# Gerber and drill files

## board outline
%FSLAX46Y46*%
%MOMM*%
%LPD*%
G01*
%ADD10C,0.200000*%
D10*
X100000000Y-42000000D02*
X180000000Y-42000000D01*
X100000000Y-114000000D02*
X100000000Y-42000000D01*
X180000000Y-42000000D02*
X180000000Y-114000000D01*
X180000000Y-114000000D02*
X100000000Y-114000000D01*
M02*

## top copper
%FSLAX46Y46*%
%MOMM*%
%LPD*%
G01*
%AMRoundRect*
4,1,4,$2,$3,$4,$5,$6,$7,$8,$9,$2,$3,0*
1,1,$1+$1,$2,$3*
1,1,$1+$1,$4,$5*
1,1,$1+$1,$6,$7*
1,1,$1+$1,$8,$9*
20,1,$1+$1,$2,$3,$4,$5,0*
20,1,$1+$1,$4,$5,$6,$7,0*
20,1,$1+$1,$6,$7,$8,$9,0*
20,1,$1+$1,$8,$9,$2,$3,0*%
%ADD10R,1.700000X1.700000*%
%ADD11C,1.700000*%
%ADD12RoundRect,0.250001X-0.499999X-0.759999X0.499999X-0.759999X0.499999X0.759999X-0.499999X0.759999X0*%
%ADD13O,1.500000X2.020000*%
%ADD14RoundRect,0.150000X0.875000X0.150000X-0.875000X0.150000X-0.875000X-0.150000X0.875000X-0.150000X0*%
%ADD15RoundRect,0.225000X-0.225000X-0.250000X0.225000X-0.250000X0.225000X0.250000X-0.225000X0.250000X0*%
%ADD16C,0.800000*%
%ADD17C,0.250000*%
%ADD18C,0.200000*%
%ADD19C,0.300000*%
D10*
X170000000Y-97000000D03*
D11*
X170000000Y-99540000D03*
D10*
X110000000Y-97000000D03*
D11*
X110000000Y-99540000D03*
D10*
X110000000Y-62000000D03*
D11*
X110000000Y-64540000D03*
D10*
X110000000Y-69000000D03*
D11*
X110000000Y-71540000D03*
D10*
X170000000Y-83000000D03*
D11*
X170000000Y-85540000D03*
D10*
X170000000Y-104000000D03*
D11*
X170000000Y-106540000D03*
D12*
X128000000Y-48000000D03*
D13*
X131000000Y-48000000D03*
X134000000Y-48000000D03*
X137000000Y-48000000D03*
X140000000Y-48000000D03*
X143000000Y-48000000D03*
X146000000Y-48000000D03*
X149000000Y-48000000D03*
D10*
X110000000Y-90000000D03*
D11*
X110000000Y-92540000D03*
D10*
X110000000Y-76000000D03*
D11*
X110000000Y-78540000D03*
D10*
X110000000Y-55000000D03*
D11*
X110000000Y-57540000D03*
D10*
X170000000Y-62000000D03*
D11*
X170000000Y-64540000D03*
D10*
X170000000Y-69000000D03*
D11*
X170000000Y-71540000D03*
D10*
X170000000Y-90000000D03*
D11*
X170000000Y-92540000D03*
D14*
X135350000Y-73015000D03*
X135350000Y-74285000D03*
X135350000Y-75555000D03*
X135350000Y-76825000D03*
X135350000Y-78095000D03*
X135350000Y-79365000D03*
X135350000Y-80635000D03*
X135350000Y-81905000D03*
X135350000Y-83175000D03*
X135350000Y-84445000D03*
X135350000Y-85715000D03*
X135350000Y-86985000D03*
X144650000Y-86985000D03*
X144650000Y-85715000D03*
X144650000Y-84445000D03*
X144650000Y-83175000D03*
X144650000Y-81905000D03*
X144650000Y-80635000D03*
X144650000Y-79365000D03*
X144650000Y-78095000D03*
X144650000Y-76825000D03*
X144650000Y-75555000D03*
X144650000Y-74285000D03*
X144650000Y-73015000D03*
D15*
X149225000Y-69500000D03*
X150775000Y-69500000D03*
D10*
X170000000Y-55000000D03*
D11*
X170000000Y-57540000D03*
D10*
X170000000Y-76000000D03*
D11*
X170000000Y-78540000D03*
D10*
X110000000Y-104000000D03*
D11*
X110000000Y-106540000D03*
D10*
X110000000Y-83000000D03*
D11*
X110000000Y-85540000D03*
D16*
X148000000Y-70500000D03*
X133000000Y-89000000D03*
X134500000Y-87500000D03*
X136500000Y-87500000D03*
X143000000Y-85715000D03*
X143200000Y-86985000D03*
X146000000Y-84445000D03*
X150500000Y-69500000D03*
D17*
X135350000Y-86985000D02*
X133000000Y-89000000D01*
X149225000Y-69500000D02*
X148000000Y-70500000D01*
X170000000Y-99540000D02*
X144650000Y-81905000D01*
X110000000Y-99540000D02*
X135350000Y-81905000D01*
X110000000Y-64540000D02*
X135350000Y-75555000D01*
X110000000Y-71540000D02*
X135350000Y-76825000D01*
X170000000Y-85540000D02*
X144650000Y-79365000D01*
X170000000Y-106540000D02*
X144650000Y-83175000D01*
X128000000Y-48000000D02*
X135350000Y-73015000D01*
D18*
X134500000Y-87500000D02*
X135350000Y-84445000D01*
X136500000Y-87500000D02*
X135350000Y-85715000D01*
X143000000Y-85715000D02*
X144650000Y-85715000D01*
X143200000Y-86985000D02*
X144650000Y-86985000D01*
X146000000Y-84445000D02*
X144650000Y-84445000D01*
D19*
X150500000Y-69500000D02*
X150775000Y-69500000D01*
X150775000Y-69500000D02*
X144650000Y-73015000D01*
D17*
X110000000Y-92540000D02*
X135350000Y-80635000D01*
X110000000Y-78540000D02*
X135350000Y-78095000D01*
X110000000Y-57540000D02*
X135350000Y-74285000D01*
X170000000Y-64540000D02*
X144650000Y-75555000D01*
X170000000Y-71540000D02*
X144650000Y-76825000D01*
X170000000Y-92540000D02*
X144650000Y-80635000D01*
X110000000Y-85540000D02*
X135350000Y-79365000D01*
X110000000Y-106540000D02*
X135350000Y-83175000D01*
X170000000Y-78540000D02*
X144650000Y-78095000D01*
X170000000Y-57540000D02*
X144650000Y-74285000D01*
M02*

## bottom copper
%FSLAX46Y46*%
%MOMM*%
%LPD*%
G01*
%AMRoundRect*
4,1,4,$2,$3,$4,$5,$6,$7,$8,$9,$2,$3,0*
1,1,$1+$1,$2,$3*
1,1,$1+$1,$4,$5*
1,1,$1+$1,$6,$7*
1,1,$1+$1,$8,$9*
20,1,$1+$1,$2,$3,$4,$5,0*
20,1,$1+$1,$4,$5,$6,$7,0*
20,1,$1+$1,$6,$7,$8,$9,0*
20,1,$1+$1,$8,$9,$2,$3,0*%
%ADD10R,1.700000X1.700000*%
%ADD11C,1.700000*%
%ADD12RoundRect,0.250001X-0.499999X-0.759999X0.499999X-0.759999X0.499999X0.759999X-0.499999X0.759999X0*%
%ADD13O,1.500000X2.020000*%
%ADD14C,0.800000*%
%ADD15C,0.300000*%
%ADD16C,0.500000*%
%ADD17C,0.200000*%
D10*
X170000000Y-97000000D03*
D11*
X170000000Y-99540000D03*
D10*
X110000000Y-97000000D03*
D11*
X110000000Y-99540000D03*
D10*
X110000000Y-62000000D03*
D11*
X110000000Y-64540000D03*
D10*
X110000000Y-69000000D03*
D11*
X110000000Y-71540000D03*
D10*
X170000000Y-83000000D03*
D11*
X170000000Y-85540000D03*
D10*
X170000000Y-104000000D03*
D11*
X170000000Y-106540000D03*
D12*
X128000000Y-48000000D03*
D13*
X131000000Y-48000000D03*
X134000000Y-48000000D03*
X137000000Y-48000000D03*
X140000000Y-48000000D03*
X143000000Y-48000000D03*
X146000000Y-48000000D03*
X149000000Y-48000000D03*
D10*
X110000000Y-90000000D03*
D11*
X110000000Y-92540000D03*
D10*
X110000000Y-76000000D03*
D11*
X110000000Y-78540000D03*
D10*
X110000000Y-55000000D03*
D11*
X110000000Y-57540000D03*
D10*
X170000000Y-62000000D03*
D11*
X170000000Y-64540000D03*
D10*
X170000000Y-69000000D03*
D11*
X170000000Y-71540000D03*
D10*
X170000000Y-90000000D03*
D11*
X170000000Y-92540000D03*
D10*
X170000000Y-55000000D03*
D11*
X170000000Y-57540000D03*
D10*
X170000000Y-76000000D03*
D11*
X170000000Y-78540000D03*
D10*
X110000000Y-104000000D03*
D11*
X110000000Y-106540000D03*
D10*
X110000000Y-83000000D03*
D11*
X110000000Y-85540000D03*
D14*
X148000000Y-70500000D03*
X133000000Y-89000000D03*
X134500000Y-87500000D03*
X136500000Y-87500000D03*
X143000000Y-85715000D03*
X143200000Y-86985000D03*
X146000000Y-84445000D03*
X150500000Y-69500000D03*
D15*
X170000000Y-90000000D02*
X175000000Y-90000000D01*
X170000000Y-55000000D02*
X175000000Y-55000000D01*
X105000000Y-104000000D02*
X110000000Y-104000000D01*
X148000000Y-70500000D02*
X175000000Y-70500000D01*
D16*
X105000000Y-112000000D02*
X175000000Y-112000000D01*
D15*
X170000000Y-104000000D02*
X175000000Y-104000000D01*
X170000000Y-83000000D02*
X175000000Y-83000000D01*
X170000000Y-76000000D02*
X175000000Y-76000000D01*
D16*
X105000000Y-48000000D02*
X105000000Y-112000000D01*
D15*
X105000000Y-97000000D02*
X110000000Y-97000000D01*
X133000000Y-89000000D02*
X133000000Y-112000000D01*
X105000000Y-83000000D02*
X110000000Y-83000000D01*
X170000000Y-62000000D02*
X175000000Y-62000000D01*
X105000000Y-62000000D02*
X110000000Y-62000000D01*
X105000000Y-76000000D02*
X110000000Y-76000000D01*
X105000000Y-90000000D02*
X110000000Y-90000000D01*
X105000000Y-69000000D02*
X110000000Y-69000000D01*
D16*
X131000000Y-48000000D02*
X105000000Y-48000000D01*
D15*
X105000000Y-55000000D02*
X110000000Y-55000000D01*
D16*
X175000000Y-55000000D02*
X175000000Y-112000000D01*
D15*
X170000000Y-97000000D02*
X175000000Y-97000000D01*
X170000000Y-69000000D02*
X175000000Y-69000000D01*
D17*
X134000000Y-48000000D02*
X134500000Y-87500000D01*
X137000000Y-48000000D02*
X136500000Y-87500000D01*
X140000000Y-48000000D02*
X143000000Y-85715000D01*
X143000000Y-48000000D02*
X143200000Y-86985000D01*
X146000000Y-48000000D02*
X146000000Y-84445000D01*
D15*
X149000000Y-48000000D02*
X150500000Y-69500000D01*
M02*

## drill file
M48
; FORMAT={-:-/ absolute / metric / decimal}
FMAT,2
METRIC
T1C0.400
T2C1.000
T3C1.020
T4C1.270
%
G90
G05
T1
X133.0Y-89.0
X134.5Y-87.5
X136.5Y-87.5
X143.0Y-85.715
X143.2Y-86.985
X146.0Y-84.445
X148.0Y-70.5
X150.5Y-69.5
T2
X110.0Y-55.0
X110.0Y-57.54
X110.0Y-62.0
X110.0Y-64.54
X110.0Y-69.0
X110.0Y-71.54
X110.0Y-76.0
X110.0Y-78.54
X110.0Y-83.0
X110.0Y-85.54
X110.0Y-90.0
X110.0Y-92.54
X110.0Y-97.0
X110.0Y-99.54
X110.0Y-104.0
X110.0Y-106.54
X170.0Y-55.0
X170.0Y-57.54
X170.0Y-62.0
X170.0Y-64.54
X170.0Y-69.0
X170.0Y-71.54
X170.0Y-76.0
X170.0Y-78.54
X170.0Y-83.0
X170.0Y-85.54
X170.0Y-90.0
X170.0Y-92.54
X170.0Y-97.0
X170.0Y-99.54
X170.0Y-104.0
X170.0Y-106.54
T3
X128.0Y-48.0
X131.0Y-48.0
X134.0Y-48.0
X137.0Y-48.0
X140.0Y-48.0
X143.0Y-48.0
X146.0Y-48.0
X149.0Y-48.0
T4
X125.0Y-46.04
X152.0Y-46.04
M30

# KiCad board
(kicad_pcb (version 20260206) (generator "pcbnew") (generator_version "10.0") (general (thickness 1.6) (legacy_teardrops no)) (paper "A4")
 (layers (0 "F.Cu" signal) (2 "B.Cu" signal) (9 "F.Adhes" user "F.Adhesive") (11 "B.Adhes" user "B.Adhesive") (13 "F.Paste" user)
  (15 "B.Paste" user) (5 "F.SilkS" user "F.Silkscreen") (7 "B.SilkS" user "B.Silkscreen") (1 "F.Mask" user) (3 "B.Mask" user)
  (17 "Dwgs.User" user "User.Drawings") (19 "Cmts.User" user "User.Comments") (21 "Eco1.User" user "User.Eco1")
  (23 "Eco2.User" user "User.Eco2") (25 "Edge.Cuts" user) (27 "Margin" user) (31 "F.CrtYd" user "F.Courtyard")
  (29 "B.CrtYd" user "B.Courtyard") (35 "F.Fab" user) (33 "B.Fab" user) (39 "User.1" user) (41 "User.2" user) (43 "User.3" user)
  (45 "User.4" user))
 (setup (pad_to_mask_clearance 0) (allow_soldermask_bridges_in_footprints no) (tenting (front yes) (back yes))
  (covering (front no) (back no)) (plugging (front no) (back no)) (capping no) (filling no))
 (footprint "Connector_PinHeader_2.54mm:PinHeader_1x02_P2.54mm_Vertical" (layer "F.Cu") (at 170 97)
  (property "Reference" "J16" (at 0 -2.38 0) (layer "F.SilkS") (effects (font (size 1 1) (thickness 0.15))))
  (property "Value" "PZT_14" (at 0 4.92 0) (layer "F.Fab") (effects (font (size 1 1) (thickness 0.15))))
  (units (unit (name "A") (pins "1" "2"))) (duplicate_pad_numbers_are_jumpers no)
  (pad "1" thru_hole rect (at 0 0) (size 1.7 1.7) (drill 1) (layers "*.Cu" "*.Mask") (remove_unused_layers no) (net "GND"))
  (pad "2" thru_hole circle (at 0 2.54) (size 1.7 1.7) (drill 1) (layers "*.Cu" "*.Mask") (remove_unused_layers no) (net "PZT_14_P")))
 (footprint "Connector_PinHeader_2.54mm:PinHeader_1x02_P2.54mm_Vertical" (layer "F.Cu") (at 110 97)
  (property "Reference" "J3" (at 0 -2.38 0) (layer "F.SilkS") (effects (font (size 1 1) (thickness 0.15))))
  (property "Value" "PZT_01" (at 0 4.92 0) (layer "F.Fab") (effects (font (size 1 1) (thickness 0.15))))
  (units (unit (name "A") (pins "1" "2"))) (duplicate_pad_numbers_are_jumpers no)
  (pad "1" thru_hole rect (at 0 0) (size 1.7 1.7) (drill 1) (layers "*.Cu" "*.Mask") (remove_unused_layers no) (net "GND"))
  (pad "2" thru_hole circle (at 0 2.54) (size 1.7 1.7) (drill 1) (layers "*.Cu" "*.Mask") (remove_unused_layers no) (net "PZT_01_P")))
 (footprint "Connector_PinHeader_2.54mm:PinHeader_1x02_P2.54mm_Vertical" (layer "F.Cu") (at 110 62)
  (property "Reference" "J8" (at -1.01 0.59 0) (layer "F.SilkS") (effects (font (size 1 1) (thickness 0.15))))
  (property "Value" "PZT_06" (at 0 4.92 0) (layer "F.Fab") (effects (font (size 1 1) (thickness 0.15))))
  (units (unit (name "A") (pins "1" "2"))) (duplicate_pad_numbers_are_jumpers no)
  (pad "1" thru_hole rect (at 0 0) (size 1.7 1.7) (drill 1) (layers "*.Cu" "*.Mask") (remove_unused_layers no) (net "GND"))
  (pad "2" thru_hole circle (at 0 2.54) (size 1.7 1.7) (drill 1) (layers "*.Cu" "*.Mask") (remove_unused_layers no) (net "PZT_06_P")))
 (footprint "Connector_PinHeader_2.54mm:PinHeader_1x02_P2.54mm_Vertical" (layer "F.Cu") (at 110 69)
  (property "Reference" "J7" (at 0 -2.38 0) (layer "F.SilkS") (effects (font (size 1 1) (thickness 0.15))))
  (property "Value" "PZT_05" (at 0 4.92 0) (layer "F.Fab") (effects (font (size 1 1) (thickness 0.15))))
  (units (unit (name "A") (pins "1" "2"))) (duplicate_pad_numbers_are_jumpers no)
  (pad "1" thru_hole rect (at 0 0) (size 1.7 1.7) (drill 1) (layers "*.Cu" "*.Mask") (remove_unused_layers no) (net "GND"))
  (pad "2" thru_hole circle (at 0 2.54) (size 1.7 1.7) (drill 1) (layers "*.Cu" "*.Mask") (remove_unused_layers no) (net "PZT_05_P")))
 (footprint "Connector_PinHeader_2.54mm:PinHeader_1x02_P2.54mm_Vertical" (layer "F.Cu") (at 170 83)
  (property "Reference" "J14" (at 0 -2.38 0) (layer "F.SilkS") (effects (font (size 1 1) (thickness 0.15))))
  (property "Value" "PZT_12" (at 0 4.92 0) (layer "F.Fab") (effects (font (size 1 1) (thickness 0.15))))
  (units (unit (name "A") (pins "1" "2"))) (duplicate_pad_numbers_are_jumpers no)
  (pad "1" thru_hole rect (at 0 0) (size 1.7 1.7) (drill 1) (layers "*.Cu" "*.Mask") (remove_unused_layers no) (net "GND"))
  (pad "2" thru_hole circle (at 0 2.54) (size 1.7 1.7) (drill 1) (layers "*.Cu" "*.Mask") (remove_unused_layers no) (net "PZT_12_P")))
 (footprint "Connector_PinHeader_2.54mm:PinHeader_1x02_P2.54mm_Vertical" (layer "F.Cu") (at 170 104)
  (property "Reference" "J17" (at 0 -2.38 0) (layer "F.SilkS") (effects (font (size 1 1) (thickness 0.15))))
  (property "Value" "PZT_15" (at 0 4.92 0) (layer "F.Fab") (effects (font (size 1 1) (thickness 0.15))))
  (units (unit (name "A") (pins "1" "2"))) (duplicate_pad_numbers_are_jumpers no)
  (pad "1" thru_hole rect (at 0 0) (size 1.7 1.7) (drill 1) (layers "*.Cu" "*.Mask") (remove_unused_layers no) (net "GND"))
  (pad "2" thru_hole circle (at 0 2.54) (size 1.7 1.7) (drill 1) (layers "*.Cu" "*.Mask") (remove_unused_layers no) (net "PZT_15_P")))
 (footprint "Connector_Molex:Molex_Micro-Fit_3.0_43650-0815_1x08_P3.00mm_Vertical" (layer "F.Cu") (at 128 48)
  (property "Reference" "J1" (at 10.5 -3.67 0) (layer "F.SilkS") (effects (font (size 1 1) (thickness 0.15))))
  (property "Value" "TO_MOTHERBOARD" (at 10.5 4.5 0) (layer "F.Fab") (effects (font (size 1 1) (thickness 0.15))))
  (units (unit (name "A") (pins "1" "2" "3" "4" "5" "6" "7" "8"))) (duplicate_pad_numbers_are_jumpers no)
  (pad "" np_thru_hole circle (at -3 -1.96) (size 1.27 1.27) (drill 1.27) (layers "*.Cu" "*.Mask"))
  (pad "" np_thru_hole circle (at 24 -1.96) (size 1.27 1.27) (drill 1.27) (layers "*.Cu" "*.Mask"))
  (pad "1" thru_hole roundrect (at 0 0) (size 1.5 2.02) (drill 1.02) (layers "*.Cu" "*.Mask") (remove_unused_layers no)
   (roundrect_rratio 0.166667) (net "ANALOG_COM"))
  (pad "2" thru_hole oval (at 3 0) (size 1.5 2.02) (drill 1.02) (layers "*.Cu" "*.Mask") (remove_unused_layers no) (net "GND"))
  (pad "3" thru_hole oval (at 6 0) (size 1.5 2.02) (drill 1.02) (layers "*.Cu" "*.Mask") (remove_unused_layers no) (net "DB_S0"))
  (pad "4" thru_hole oval (at 9 0) (size 1.5 2.02) (drill 1.02) (layers "*.Cu" "*.Mask") (remove_unused_layers no) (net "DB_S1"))
  (pad "5" thru_hole oval (at 12 0) (size 1.5 2.02) (drill 1.02) (layers "*.Cu" "*.Mask") (remove_unused_layers no) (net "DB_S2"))
  (pad "6" thru_hole oval (at 15 0) (size 1.5 2.02) (drill 1.02) (layers "*.Cu" "*.Mask") (remove_unused_layers no) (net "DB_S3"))
  (pad "7" thru_hole oval (at 18 0) (size 1.5 2.02) (drill 1.02) (layers "*.Cu" "*.Mask") (remove_unused_layers no) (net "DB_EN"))
  (pad "8" thru_hole oval (at 21 0) (size 1.5 2.02) (drill 1.02) (layers "*.Cu" "*.Mask") (remove_unused_layers no) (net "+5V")))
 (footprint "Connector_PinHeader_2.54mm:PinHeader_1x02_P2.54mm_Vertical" (layer "F.Cu") (at 110 90)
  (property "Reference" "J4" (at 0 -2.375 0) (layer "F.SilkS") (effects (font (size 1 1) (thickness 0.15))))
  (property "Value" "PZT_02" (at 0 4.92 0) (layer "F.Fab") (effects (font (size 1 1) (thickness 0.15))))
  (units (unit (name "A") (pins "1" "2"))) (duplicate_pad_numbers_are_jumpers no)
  (pad "1" thru_hole rect (at 0 0) (size 1.7 1.7) (drill 1) (layers "*.Cu" "*.Mask") (remove_unused_layers no) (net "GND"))
  (pad "2" thru_hole circle (at 0 2.54) (size 1.7 1.7) (drill 1) (layers "*.Cu" "*.Mask") (remove_unused_layers no) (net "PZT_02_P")))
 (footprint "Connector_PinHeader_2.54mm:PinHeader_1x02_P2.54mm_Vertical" (layer "F.Cu") (at 110 76)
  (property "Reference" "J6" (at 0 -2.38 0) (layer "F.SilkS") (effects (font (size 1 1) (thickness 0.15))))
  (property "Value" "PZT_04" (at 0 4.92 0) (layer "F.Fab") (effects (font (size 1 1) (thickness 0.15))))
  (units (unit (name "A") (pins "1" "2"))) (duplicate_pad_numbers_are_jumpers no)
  (pad "1" thru_hole rect (at 0 0) (size 1.7 1.7) (drill 1) (layers "*.Cu" "*.Mask") (remove_unused_layers no) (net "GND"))
  (pad "2" thru_hole circle (at 0 2.54) (size 1.7 1.7) (drill 1) (layers "*.Cu" "*.Mask") (remove_unused_layers no) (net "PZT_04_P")))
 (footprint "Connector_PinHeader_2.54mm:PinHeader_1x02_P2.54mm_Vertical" (layer "F.Cu") (at 110 55)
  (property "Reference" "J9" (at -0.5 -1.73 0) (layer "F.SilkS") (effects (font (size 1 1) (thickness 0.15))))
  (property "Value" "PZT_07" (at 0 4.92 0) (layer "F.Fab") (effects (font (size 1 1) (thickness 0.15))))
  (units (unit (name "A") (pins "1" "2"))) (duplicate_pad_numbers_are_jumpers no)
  (pad "1" thru_hole rect (at 0 0) (size 1.7 1.7) (drill 1) (layers "*.Cu" "*.Mask") (remove_unused_layers no) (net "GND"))
  (pad "2" thru_hole circle (at 0 2.54) (size 1.7 1.7) (drill 1) (layers "*.Cu" "*.Mask") (remove_unused_layers no) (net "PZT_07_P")))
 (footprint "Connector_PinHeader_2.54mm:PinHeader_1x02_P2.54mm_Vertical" (layer "F.Cu") (at 170 62)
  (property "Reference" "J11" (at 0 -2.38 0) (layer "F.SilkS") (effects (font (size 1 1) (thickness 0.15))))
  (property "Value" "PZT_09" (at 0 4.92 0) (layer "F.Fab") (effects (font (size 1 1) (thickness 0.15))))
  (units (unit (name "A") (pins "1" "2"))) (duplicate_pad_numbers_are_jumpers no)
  (pad "1" thru_hole rect (at 0 0) (size 1.7 1.7) (drill 1) (layers "*.Cu" "*.Mask") (remove_unused_layers no) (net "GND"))
  (pad "2" thru_hole circle (at 0 2.54) (size 1.7 1.7) (drill 1) (layers "*.Cu" "*.Mask") (remove_unused_layers no) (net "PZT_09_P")))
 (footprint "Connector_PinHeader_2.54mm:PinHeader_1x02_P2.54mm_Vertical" (layer "F.Cu") (at 170 69)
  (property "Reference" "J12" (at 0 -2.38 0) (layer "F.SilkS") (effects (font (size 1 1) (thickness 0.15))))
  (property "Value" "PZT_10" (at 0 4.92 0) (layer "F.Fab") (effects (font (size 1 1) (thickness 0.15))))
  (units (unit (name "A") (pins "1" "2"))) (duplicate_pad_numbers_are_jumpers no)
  (pad "1" thru_hole rect (at 0 0) (size 1.7 1.7) (drill 1) (layers "*.Cu" "*.Mask") (remove_unused_layers no) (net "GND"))
  (pad "2" thru_hole circle (at 0 2.54) (size 1.7 1.7) (drill 1) (layers "*.Cu" "*.Mask") (remove_unused_layers no) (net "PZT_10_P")))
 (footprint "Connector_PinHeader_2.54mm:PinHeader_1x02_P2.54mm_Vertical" (layer "F.Cu") (at 170 90)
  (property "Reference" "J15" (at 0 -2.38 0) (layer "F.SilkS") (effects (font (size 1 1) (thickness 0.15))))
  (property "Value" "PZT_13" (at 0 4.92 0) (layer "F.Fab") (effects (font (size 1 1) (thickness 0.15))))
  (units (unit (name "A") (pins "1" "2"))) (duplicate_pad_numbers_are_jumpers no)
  (pad "1" thru_hole rect (at 0 0) (size 1.7 1.7) (drill 1) (layers "*.Cu" "*.Mask") (remove_unused_layers no) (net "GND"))
  (pad "2" thru_hole circle (at 0 2.54) (size 1.7 1.7) (drill 1) (layers "*.Cu" "*.Mask") (remove_unused_layers no) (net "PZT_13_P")))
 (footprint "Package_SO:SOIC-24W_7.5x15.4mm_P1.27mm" (layer "F.Cu") (at 140 80)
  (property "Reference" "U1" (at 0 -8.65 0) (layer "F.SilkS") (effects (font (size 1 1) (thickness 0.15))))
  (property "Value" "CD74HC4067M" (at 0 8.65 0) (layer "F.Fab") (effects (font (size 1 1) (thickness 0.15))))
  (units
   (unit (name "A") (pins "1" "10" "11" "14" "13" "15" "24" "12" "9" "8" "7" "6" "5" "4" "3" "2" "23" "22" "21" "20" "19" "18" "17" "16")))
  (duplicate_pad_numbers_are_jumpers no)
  (pad "1" smd roundrect (at -4.65 -6.985 180) (size 2.05 0.6) (layers "F.Cu" "F.Mask" "F.Paste") (roundrect_rratio 0.25) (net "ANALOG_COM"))
  (pad "2" smd roundrect (at -4.65 -5.715 180) (size 2.05 0.6) (layers "F.Cu" "F.Mask" "F.Paste") (roundrect_rratio 0.25) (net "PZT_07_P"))
  (pad "3" smd roundrect (at -4.65 -4.445 180) (size 2.05 0.6) (layers "F.Cu" "F.Mask" "F.Paste") (roundrect_rratio 0.25) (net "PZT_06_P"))
  (pad "4" smd roundrect (at -4.65 -3.175 180) (size 2.05 0.6) (layers "F.Cu" "F.Mask" "F.Paste") (roundrect_rratio 0.25) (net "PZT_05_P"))
  (pad "5" smd roundrect (at -4.65 -1.905 180) (size 2.05 0.6) (layers "F.Cu" "F.Mask" "F.Paste") (roundrect_rratio 0.25) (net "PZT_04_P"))
  (pad "6" smd roundrect (at -4.65 -0.635 180) (size 2.05 0.6) (layers "F.Cu" "F.Mask" "F.Paste") (roundrect_rratio 0.25) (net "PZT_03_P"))
  (pad "7" smd roundrect (at -4.65 0.635 180) (size 2.05 0.6) (layers "F.Cu" "F.Mask" "F.Paste") (roundrect_rratio 0.25) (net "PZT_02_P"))
  (pad "8" smd roundrect (at -4.65 1.905 180) (size 2.05 0.6) (layers "F.Cu" "F.Mask" "F.Paste") (roundrect_rratio 0.25) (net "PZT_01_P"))
  (pad "9" smd roundrect (at -4.65 3.175 180) (size 2.05 0.6) (layers "F.Cu" "F.Mask" "F.Paste") (roundrect_rratio 0.25) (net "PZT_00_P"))
  (pad "10" smd roundrect (at -4.65 4.445 180) (size 2.05 0.6) (layers "F.Cu" "F.Mask" "F.Paste") (roundrect_rratio 0.25) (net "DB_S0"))
  (pad "11" smd roundrect (at -4.65 5.715 180) (size 2.05 0.6) (layers "F.Cu" "F.Mask" "F.Paste") (roundrect_rratio 0.25) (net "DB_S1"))
  (pad "12" smd roundrect (at -4.65 6.985 180) (size 2.05 0.6) (layers "F.Cu" "F.Mask" "F.Paste") (roundrect_rratio 0.25) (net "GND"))
  (pad "13" smd roundrect (at 4.65 6.985 180) (size 2.05 0.6) (layers "F.Cu" "F.Mask" "F.Paste") (roundrect_rratio 0.25) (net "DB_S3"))
  (pad "14" smd roundrect (at 4.65 5.715 180) (size 2.05 0.6) (layers "F.Cu" "F.Mask" "F.Paste") (roundrect_rratio 0.25) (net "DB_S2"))
  (pad "15" smd roundrect (at 4.65 4.445 180) (size 2.05 0.6) (layers "F.Cu" "F.Mask" "F.Paste") (roundrect_rratio 0.25) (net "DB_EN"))
  (pad "16" smd roundrect (at 4.65 3.175 180) (size 2.05 0.6) (layers "F.Cu" "F.Mask" "F.Paste") (roundrect_rratio 0.25) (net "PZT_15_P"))
  (pad "17" smd roundrect (at 4.65 1.905 180) (size 2.05 0.6) (layers "F.Cu" "F.Mask" "F.Paste") (roundrect_rratio 0.25) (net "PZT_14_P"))
  (pad "18" smd roundrect (at 4.65 0.635 180) (size 2.05 0.6) (layers "F.Cu" "F.Mask" "F.Paste") (roundrect_rratio 0.25) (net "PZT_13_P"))
  (pad "19" smd roundrect (at 4.65 -0.635 180) (size 2.05 0.6) (layers "F.Cu" "F.Mask" "F.Paste") (roundrect_rratio 0.25) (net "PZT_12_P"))
  (pad "20" smd roundrect (at 4.65 -1.905 180) (size 2.05 0.6) (layers "F.Cu" "F.Mask" "F.Paste") (roundrect_rratio 0.25) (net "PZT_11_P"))
  (pad "21" smd roundrect (at 4.65 -3.175 180) (size 2.05 0.6) (layers "F.Cu" "F.Mask" "F.Paste") (roundrect_rratio 0.25) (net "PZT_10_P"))
  (pad "22" smd roundrect (at 4.65 -4.445 180) (size 2.05 0.6) (layers "F.Cu" "F.Mask" "F.Paste") (roundrect_rratio 0.25) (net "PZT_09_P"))
  (pad "23" smd roundrect (at 4.65 -5.715 180) (size 2.05 0.6) (layers "F.Cu" "F.Mask" "F.Paste") (roundrect_rratio 0.25) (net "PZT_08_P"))
  (pad "24" smd roundrect (at 4.65 -6.985 180) (size 2.05 0.6) (layers "F.Cu" "F.Mask" "F.Paste") (roundrect_rratio 0.25) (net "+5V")))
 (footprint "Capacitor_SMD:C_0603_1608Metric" (layer "F.Cu") (at 150 69.5)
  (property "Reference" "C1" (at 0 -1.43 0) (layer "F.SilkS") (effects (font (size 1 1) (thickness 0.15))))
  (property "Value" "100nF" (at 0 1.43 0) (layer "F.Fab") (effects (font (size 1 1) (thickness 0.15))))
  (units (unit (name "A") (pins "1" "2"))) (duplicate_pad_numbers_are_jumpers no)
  (pad "1" smd roundrect (at -0.775 0) (size 0.9 0.95) (layers "F.Cu" "F.Mask" "F.Paste") (roundrect_rratio 0.25) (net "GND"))
  (pad "2" smd roundrect (at 0.775 0) (size 0.9 0.95) (layers "F.Cu" "F.Mask" "F.Paste") (roundrect_rratio 0.25) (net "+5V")))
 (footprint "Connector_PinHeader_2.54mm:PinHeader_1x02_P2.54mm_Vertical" (layer "F.Cu") (at 170 55)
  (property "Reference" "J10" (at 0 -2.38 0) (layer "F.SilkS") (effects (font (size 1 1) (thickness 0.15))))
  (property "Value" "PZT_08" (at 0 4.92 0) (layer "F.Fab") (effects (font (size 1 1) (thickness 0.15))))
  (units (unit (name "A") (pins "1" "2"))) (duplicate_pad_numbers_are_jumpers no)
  (pad "1" thru_hole rect (at 0 0) (size 1.7 1.7) (drill 1) (layers "*.Cu" "*.Mask") (remove_unused_layers no) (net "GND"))
  (pad "2" thru_hole circle (at 0 2.54) (size 1.7 1.7) (drill 1) (layers "*.Cu" "*.Mask") (remove_unused_layers no) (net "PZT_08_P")))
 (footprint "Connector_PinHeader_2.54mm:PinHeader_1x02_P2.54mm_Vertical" (layer "F.Cu") (at 170 76)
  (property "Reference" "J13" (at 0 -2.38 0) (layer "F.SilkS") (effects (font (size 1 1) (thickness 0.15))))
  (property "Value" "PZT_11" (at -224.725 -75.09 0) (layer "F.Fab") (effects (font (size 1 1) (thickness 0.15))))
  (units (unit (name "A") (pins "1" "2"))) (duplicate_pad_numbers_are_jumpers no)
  (pad "1" thru_hole rect (at 0 0) (size 1.7 1.7) (drill 1) (layers "*.Cu" "*.Mask") (remove_unused_layers no) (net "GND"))
  (pad "2" thru_hole circle (at 0 2.54) (size 1.7 1.7) (drill 1) (layers "*.Cu" "*.Mask") (remove_unused_layers no) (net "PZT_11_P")))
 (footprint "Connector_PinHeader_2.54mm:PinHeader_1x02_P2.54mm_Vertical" (layer "F.Cu") (at 110 104)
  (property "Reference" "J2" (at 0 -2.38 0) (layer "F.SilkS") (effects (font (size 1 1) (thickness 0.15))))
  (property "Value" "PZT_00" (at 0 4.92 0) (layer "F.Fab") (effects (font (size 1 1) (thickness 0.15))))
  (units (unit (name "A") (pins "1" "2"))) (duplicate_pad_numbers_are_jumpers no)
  (pad "1" thru_hole rect (at 0 0) (size 1.7 1.7) (drill 1) (layers "*.Cu" "*.Mask") (remove_unused_layers no) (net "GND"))
  (pad "2" thru_hole circle (at 0 2.54) (size 1.7 1.7) (drill 1) (layers "*.Cu" "*.Mask") (remove_unused_layers no) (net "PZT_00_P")))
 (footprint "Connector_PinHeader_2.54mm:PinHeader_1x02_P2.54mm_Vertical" (layer "F.Cu") (at 110 83)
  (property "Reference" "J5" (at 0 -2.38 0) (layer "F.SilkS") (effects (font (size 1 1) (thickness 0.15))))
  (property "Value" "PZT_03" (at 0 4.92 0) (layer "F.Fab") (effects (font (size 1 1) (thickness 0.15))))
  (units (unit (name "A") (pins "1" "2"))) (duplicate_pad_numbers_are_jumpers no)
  (pad "1" thru_hole rect (at 0 0) (size 1.7 1.7) (drill 1) (layers "*.Cu" "*.Mask") (remove_unused_layers no) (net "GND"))
  (pad "2" thru_hole circle (at 0 2.54) (size 1.7 1.7) (drill 1) (layers "*.Cu" "*.Mask") (remove_unused_layers no) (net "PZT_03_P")))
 (gr_line (start 100 42) (end 180 42) (stroke (width 0.2) (type solid)) (layer "Edge.Cuts"))
 (gr_line (start 100 114) (end 100 42) (stroke (width 0.2) (type solid)) (layer "Edge.Cuts"))
 (gr_line (start 180 42) (end 180 114) (stroke (width 0.2) (type solid)) (layer "Edge.Cuts"))
 (gr_line (start 180 114) (end 100 114) (stroke (width 0.2) (type solid)) (layer "Edge.Cuts"))
 (segment (start 135.35 86.985) (end 133 89) (width 0.25) (layer "F.Cu") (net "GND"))
 (segment (start 149.225 69.5) (end 148 70.5) (width 0.25) (layer "F.Cu") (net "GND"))
 (via (at 148 70.5) (size 0.8) (drill 0.4) (layers "F.Cu" "B.Cu") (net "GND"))
 (via (at 133 89) (size 0.8) (drill 0.4) (layers "F.Cu" "B.Cu") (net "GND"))
 (segment (start 170 90) (end 175 90) (width 0.3) (layer "B.Cu") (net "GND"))
 (segment (start 170 55) (end 175 55) (width 0.3) (layer "B.Cu") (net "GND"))
 (segment (start 105 104) (end 110 104) (width 0.3) (layer "B.Cu") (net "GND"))
 (segment (start 148 70.5) (end 175 70.5) (width 0.3) (layer "B.Cu") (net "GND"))
 (segment (start 105 112) (end 175 112) (width 0.5) (layer "B.Cu") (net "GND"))
 (segment (start 170 104) (end 175 104) (width 0.3) (layer "B.Cu") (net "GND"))
 (segment (start 170 83) (end 175 83) (width 0.3) (layer "B.Cu") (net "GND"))
 (segment (start 170 76) (end 175 76) (width 0.3) (layer "B.Cu") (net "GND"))
 (segment (start 105 48) (end 105 112) (width 0.5) (layer "B.Cu") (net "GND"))
 (segment (start 105 97) (end 110 97) (width 0.3) (layer "B.Cu") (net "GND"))
 (segment (start 133 89) (end 133 112) (width 0.3) (layer "B.Cu") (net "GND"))
 (segment (start 105 83) (end 110 83) (width 0.3) (layer "B.Cu") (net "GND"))
 (segment (start 170 62) (end 175 62) (width 0.3) (layer "B.Cu") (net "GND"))
 (segment (start 105 62) (end 110 62) (width 0.3) (layer "B.Cu") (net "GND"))
 (segment (start 105 76) (end 110 76) (width 0.3) (layer "B.Cu") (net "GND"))
 (segment (start 105 90) (end 110 90) (width 0.3) (layer "B.Cu") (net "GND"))
 (segment (start 105 69) (end 110 69) (width 0.3) (layer "B.Cu") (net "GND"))
 (segment (start 131 48) (end 105 48) (width 0.5) (layer "B.Cu") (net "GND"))
 (segment (start 105 55) (end 110 55) (width 0.3) (layer "B.Cu") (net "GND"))
 (segment (start 175 55) (end 175 112) (width 0.5) (layer "B.Cu") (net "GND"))
 (segment (start 170 97) (end 175 97) (width 0.3) (layer "B.Cu") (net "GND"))
 (segment (start 170 69) (end 175 69) (width 0.3) (layer "B.Cu") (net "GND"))
 (segment (start 170 99.54) (end 144.65 81.905) (width 0.25) (layer "F.Cu") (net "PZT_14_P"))
 (segment (start 110 99.54) (end 135.35 81.905) (width 0.25) (layer "F.Cu") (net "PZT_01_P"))
 (segment (start 110 64.54) (end 135.35 75.555) (width 0.25) (layer "F.Cu") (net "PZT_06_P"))
 (segment (start 110 71.54) (end 135.35 76.825) (width 0.25) (layer "F.Cu") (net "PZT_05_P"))
 (segment (start 170 85.54) (end 144.65 79.365) (width 0.25) (layer "F.Cu") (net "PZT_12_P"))
 (segment (start 170 106.54) (end 144.65 83.175) (width 0.25) (layer "F.Cu") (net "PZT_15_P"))
 (segment (start 128 48) (end 135.35 73.015) (width 0.25) (layer "F.Cu") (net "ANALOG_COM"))
 (segment (start 134.5 87.5) (end 135.35 84.445) (width 0.2) (layer "F.Cu") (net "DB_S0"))
 (via (at 134.5 87.5) (size 0.8) (drill 0.4) (layers "F.Cu" "B.Cu") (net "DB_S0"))
 (segment (start 134 48) (end 134.5 87.5) (width 0.2) (layer "B.Cu") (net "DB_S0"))
 (segment (start 136.5 87.5) (end 135.35 85.715) (width 0.2) (layer "F.Cu") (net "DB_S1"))
 (via (at 136.5 87.5) (size 0.8) (drill 0.4) (layers "F.Cu" "B.Cu") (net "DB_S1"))
 (segment (start 137 48) (end 136.5 87.5) (width 0.2) (layer "B.Cu") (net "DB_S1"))
 (segment (start 143 85.715) (end 144.65 85.715) (width 0.2) (layer "F.Cu") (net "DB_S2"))
 (via (at 143 85.715) (size 0.8) (drill 0.4) (layers "F.Cu" "B.Cu") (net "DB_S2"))
 (segment (start 140 48) (end 143 85.715) (width 0.2) (layer "B.Cu") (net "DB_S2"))
 (segment (start 143.2 86.985) (end 144.65 86.985) (width 0.2) (layer "F.Cu") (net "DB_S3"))
 (via (at 143.2 86.985) (size 0.8) (drill 0.4) (layers "F.Cu" "B.Cu") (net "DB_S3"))
 (segment (start 143 48) (end 143.2 86.985) (width 0.2) (layer "B.Cu") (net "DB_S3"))
 (segment (start 146 84.445) (end 144.65 84.445) (width 0.2) (layer "F.Cu") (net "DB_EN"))
 (via (at 146 84.445) (size 0.8) (drill 0.4) (layers "F.Cu" "B.Cu") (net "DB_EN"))
 (segment (start 146 48) (end 146 84.445) (width 0.2) (layer "B.Cu") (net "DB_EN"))
 (segment (start 150.5 69.5) (end 150.775 69.5) (width 0.3) (layer "F.Cu") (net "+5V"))
 (segment (start 150.775 69.5) (end 144.65 73.015) (width 0.3) (layer "F.Cu") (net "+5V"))
 (via (at 150.5 69.5) (size 0.8) (drill 0.4) (layers "F.Cu" "B.Cu") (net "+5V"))
 (segment (start 149 48) (end 150.5 69.5) (width 0.3) (layer "B.Cu") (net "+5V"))
 (segment (start 110 92.54) (end 135.35 80.635) (width 0.25) (layer "F.Cu") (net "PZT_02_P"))
 (segment (start 110 78.54) (end 135.35 78.095) (width 0.25) (layer "F.Cu") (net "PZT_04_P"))
 (segment (start 110 57.54) (end 135.35 74.285) (width 0.25) (layer "F.Cu") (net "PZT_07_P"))
 (segment (start 170 64.54) (end 144.65 75.555) (width 0.25) (layer "F.Cu") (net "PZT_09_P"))
 (segment (start 170 71.54) (end 144.65 76.825) (width 0.25) (layer "F.Cu") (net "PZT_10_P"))
 (segment (start 170 92.54) (end 144.65 80.635) (width 0.25) (layer "F.Cu") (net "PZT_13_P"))
 (segment (start 110 85.54) (end 135.35 79.365) (width 0.25) (layer "F.Cu") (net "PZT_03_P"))
 (segment (start 110 106.54) (end 135.35 83.175) (width 0.25) (layer "F.Cu") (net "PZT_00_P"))
 (segment (start 170 78.54) (end 144.65 78.095) (width 0.25) (layer "F.Cu") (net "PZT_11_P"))
 (segment (start 170 57.54) (end 144.65 74.285) (width 0.25) (layer "F.Cu") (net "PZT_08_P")))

